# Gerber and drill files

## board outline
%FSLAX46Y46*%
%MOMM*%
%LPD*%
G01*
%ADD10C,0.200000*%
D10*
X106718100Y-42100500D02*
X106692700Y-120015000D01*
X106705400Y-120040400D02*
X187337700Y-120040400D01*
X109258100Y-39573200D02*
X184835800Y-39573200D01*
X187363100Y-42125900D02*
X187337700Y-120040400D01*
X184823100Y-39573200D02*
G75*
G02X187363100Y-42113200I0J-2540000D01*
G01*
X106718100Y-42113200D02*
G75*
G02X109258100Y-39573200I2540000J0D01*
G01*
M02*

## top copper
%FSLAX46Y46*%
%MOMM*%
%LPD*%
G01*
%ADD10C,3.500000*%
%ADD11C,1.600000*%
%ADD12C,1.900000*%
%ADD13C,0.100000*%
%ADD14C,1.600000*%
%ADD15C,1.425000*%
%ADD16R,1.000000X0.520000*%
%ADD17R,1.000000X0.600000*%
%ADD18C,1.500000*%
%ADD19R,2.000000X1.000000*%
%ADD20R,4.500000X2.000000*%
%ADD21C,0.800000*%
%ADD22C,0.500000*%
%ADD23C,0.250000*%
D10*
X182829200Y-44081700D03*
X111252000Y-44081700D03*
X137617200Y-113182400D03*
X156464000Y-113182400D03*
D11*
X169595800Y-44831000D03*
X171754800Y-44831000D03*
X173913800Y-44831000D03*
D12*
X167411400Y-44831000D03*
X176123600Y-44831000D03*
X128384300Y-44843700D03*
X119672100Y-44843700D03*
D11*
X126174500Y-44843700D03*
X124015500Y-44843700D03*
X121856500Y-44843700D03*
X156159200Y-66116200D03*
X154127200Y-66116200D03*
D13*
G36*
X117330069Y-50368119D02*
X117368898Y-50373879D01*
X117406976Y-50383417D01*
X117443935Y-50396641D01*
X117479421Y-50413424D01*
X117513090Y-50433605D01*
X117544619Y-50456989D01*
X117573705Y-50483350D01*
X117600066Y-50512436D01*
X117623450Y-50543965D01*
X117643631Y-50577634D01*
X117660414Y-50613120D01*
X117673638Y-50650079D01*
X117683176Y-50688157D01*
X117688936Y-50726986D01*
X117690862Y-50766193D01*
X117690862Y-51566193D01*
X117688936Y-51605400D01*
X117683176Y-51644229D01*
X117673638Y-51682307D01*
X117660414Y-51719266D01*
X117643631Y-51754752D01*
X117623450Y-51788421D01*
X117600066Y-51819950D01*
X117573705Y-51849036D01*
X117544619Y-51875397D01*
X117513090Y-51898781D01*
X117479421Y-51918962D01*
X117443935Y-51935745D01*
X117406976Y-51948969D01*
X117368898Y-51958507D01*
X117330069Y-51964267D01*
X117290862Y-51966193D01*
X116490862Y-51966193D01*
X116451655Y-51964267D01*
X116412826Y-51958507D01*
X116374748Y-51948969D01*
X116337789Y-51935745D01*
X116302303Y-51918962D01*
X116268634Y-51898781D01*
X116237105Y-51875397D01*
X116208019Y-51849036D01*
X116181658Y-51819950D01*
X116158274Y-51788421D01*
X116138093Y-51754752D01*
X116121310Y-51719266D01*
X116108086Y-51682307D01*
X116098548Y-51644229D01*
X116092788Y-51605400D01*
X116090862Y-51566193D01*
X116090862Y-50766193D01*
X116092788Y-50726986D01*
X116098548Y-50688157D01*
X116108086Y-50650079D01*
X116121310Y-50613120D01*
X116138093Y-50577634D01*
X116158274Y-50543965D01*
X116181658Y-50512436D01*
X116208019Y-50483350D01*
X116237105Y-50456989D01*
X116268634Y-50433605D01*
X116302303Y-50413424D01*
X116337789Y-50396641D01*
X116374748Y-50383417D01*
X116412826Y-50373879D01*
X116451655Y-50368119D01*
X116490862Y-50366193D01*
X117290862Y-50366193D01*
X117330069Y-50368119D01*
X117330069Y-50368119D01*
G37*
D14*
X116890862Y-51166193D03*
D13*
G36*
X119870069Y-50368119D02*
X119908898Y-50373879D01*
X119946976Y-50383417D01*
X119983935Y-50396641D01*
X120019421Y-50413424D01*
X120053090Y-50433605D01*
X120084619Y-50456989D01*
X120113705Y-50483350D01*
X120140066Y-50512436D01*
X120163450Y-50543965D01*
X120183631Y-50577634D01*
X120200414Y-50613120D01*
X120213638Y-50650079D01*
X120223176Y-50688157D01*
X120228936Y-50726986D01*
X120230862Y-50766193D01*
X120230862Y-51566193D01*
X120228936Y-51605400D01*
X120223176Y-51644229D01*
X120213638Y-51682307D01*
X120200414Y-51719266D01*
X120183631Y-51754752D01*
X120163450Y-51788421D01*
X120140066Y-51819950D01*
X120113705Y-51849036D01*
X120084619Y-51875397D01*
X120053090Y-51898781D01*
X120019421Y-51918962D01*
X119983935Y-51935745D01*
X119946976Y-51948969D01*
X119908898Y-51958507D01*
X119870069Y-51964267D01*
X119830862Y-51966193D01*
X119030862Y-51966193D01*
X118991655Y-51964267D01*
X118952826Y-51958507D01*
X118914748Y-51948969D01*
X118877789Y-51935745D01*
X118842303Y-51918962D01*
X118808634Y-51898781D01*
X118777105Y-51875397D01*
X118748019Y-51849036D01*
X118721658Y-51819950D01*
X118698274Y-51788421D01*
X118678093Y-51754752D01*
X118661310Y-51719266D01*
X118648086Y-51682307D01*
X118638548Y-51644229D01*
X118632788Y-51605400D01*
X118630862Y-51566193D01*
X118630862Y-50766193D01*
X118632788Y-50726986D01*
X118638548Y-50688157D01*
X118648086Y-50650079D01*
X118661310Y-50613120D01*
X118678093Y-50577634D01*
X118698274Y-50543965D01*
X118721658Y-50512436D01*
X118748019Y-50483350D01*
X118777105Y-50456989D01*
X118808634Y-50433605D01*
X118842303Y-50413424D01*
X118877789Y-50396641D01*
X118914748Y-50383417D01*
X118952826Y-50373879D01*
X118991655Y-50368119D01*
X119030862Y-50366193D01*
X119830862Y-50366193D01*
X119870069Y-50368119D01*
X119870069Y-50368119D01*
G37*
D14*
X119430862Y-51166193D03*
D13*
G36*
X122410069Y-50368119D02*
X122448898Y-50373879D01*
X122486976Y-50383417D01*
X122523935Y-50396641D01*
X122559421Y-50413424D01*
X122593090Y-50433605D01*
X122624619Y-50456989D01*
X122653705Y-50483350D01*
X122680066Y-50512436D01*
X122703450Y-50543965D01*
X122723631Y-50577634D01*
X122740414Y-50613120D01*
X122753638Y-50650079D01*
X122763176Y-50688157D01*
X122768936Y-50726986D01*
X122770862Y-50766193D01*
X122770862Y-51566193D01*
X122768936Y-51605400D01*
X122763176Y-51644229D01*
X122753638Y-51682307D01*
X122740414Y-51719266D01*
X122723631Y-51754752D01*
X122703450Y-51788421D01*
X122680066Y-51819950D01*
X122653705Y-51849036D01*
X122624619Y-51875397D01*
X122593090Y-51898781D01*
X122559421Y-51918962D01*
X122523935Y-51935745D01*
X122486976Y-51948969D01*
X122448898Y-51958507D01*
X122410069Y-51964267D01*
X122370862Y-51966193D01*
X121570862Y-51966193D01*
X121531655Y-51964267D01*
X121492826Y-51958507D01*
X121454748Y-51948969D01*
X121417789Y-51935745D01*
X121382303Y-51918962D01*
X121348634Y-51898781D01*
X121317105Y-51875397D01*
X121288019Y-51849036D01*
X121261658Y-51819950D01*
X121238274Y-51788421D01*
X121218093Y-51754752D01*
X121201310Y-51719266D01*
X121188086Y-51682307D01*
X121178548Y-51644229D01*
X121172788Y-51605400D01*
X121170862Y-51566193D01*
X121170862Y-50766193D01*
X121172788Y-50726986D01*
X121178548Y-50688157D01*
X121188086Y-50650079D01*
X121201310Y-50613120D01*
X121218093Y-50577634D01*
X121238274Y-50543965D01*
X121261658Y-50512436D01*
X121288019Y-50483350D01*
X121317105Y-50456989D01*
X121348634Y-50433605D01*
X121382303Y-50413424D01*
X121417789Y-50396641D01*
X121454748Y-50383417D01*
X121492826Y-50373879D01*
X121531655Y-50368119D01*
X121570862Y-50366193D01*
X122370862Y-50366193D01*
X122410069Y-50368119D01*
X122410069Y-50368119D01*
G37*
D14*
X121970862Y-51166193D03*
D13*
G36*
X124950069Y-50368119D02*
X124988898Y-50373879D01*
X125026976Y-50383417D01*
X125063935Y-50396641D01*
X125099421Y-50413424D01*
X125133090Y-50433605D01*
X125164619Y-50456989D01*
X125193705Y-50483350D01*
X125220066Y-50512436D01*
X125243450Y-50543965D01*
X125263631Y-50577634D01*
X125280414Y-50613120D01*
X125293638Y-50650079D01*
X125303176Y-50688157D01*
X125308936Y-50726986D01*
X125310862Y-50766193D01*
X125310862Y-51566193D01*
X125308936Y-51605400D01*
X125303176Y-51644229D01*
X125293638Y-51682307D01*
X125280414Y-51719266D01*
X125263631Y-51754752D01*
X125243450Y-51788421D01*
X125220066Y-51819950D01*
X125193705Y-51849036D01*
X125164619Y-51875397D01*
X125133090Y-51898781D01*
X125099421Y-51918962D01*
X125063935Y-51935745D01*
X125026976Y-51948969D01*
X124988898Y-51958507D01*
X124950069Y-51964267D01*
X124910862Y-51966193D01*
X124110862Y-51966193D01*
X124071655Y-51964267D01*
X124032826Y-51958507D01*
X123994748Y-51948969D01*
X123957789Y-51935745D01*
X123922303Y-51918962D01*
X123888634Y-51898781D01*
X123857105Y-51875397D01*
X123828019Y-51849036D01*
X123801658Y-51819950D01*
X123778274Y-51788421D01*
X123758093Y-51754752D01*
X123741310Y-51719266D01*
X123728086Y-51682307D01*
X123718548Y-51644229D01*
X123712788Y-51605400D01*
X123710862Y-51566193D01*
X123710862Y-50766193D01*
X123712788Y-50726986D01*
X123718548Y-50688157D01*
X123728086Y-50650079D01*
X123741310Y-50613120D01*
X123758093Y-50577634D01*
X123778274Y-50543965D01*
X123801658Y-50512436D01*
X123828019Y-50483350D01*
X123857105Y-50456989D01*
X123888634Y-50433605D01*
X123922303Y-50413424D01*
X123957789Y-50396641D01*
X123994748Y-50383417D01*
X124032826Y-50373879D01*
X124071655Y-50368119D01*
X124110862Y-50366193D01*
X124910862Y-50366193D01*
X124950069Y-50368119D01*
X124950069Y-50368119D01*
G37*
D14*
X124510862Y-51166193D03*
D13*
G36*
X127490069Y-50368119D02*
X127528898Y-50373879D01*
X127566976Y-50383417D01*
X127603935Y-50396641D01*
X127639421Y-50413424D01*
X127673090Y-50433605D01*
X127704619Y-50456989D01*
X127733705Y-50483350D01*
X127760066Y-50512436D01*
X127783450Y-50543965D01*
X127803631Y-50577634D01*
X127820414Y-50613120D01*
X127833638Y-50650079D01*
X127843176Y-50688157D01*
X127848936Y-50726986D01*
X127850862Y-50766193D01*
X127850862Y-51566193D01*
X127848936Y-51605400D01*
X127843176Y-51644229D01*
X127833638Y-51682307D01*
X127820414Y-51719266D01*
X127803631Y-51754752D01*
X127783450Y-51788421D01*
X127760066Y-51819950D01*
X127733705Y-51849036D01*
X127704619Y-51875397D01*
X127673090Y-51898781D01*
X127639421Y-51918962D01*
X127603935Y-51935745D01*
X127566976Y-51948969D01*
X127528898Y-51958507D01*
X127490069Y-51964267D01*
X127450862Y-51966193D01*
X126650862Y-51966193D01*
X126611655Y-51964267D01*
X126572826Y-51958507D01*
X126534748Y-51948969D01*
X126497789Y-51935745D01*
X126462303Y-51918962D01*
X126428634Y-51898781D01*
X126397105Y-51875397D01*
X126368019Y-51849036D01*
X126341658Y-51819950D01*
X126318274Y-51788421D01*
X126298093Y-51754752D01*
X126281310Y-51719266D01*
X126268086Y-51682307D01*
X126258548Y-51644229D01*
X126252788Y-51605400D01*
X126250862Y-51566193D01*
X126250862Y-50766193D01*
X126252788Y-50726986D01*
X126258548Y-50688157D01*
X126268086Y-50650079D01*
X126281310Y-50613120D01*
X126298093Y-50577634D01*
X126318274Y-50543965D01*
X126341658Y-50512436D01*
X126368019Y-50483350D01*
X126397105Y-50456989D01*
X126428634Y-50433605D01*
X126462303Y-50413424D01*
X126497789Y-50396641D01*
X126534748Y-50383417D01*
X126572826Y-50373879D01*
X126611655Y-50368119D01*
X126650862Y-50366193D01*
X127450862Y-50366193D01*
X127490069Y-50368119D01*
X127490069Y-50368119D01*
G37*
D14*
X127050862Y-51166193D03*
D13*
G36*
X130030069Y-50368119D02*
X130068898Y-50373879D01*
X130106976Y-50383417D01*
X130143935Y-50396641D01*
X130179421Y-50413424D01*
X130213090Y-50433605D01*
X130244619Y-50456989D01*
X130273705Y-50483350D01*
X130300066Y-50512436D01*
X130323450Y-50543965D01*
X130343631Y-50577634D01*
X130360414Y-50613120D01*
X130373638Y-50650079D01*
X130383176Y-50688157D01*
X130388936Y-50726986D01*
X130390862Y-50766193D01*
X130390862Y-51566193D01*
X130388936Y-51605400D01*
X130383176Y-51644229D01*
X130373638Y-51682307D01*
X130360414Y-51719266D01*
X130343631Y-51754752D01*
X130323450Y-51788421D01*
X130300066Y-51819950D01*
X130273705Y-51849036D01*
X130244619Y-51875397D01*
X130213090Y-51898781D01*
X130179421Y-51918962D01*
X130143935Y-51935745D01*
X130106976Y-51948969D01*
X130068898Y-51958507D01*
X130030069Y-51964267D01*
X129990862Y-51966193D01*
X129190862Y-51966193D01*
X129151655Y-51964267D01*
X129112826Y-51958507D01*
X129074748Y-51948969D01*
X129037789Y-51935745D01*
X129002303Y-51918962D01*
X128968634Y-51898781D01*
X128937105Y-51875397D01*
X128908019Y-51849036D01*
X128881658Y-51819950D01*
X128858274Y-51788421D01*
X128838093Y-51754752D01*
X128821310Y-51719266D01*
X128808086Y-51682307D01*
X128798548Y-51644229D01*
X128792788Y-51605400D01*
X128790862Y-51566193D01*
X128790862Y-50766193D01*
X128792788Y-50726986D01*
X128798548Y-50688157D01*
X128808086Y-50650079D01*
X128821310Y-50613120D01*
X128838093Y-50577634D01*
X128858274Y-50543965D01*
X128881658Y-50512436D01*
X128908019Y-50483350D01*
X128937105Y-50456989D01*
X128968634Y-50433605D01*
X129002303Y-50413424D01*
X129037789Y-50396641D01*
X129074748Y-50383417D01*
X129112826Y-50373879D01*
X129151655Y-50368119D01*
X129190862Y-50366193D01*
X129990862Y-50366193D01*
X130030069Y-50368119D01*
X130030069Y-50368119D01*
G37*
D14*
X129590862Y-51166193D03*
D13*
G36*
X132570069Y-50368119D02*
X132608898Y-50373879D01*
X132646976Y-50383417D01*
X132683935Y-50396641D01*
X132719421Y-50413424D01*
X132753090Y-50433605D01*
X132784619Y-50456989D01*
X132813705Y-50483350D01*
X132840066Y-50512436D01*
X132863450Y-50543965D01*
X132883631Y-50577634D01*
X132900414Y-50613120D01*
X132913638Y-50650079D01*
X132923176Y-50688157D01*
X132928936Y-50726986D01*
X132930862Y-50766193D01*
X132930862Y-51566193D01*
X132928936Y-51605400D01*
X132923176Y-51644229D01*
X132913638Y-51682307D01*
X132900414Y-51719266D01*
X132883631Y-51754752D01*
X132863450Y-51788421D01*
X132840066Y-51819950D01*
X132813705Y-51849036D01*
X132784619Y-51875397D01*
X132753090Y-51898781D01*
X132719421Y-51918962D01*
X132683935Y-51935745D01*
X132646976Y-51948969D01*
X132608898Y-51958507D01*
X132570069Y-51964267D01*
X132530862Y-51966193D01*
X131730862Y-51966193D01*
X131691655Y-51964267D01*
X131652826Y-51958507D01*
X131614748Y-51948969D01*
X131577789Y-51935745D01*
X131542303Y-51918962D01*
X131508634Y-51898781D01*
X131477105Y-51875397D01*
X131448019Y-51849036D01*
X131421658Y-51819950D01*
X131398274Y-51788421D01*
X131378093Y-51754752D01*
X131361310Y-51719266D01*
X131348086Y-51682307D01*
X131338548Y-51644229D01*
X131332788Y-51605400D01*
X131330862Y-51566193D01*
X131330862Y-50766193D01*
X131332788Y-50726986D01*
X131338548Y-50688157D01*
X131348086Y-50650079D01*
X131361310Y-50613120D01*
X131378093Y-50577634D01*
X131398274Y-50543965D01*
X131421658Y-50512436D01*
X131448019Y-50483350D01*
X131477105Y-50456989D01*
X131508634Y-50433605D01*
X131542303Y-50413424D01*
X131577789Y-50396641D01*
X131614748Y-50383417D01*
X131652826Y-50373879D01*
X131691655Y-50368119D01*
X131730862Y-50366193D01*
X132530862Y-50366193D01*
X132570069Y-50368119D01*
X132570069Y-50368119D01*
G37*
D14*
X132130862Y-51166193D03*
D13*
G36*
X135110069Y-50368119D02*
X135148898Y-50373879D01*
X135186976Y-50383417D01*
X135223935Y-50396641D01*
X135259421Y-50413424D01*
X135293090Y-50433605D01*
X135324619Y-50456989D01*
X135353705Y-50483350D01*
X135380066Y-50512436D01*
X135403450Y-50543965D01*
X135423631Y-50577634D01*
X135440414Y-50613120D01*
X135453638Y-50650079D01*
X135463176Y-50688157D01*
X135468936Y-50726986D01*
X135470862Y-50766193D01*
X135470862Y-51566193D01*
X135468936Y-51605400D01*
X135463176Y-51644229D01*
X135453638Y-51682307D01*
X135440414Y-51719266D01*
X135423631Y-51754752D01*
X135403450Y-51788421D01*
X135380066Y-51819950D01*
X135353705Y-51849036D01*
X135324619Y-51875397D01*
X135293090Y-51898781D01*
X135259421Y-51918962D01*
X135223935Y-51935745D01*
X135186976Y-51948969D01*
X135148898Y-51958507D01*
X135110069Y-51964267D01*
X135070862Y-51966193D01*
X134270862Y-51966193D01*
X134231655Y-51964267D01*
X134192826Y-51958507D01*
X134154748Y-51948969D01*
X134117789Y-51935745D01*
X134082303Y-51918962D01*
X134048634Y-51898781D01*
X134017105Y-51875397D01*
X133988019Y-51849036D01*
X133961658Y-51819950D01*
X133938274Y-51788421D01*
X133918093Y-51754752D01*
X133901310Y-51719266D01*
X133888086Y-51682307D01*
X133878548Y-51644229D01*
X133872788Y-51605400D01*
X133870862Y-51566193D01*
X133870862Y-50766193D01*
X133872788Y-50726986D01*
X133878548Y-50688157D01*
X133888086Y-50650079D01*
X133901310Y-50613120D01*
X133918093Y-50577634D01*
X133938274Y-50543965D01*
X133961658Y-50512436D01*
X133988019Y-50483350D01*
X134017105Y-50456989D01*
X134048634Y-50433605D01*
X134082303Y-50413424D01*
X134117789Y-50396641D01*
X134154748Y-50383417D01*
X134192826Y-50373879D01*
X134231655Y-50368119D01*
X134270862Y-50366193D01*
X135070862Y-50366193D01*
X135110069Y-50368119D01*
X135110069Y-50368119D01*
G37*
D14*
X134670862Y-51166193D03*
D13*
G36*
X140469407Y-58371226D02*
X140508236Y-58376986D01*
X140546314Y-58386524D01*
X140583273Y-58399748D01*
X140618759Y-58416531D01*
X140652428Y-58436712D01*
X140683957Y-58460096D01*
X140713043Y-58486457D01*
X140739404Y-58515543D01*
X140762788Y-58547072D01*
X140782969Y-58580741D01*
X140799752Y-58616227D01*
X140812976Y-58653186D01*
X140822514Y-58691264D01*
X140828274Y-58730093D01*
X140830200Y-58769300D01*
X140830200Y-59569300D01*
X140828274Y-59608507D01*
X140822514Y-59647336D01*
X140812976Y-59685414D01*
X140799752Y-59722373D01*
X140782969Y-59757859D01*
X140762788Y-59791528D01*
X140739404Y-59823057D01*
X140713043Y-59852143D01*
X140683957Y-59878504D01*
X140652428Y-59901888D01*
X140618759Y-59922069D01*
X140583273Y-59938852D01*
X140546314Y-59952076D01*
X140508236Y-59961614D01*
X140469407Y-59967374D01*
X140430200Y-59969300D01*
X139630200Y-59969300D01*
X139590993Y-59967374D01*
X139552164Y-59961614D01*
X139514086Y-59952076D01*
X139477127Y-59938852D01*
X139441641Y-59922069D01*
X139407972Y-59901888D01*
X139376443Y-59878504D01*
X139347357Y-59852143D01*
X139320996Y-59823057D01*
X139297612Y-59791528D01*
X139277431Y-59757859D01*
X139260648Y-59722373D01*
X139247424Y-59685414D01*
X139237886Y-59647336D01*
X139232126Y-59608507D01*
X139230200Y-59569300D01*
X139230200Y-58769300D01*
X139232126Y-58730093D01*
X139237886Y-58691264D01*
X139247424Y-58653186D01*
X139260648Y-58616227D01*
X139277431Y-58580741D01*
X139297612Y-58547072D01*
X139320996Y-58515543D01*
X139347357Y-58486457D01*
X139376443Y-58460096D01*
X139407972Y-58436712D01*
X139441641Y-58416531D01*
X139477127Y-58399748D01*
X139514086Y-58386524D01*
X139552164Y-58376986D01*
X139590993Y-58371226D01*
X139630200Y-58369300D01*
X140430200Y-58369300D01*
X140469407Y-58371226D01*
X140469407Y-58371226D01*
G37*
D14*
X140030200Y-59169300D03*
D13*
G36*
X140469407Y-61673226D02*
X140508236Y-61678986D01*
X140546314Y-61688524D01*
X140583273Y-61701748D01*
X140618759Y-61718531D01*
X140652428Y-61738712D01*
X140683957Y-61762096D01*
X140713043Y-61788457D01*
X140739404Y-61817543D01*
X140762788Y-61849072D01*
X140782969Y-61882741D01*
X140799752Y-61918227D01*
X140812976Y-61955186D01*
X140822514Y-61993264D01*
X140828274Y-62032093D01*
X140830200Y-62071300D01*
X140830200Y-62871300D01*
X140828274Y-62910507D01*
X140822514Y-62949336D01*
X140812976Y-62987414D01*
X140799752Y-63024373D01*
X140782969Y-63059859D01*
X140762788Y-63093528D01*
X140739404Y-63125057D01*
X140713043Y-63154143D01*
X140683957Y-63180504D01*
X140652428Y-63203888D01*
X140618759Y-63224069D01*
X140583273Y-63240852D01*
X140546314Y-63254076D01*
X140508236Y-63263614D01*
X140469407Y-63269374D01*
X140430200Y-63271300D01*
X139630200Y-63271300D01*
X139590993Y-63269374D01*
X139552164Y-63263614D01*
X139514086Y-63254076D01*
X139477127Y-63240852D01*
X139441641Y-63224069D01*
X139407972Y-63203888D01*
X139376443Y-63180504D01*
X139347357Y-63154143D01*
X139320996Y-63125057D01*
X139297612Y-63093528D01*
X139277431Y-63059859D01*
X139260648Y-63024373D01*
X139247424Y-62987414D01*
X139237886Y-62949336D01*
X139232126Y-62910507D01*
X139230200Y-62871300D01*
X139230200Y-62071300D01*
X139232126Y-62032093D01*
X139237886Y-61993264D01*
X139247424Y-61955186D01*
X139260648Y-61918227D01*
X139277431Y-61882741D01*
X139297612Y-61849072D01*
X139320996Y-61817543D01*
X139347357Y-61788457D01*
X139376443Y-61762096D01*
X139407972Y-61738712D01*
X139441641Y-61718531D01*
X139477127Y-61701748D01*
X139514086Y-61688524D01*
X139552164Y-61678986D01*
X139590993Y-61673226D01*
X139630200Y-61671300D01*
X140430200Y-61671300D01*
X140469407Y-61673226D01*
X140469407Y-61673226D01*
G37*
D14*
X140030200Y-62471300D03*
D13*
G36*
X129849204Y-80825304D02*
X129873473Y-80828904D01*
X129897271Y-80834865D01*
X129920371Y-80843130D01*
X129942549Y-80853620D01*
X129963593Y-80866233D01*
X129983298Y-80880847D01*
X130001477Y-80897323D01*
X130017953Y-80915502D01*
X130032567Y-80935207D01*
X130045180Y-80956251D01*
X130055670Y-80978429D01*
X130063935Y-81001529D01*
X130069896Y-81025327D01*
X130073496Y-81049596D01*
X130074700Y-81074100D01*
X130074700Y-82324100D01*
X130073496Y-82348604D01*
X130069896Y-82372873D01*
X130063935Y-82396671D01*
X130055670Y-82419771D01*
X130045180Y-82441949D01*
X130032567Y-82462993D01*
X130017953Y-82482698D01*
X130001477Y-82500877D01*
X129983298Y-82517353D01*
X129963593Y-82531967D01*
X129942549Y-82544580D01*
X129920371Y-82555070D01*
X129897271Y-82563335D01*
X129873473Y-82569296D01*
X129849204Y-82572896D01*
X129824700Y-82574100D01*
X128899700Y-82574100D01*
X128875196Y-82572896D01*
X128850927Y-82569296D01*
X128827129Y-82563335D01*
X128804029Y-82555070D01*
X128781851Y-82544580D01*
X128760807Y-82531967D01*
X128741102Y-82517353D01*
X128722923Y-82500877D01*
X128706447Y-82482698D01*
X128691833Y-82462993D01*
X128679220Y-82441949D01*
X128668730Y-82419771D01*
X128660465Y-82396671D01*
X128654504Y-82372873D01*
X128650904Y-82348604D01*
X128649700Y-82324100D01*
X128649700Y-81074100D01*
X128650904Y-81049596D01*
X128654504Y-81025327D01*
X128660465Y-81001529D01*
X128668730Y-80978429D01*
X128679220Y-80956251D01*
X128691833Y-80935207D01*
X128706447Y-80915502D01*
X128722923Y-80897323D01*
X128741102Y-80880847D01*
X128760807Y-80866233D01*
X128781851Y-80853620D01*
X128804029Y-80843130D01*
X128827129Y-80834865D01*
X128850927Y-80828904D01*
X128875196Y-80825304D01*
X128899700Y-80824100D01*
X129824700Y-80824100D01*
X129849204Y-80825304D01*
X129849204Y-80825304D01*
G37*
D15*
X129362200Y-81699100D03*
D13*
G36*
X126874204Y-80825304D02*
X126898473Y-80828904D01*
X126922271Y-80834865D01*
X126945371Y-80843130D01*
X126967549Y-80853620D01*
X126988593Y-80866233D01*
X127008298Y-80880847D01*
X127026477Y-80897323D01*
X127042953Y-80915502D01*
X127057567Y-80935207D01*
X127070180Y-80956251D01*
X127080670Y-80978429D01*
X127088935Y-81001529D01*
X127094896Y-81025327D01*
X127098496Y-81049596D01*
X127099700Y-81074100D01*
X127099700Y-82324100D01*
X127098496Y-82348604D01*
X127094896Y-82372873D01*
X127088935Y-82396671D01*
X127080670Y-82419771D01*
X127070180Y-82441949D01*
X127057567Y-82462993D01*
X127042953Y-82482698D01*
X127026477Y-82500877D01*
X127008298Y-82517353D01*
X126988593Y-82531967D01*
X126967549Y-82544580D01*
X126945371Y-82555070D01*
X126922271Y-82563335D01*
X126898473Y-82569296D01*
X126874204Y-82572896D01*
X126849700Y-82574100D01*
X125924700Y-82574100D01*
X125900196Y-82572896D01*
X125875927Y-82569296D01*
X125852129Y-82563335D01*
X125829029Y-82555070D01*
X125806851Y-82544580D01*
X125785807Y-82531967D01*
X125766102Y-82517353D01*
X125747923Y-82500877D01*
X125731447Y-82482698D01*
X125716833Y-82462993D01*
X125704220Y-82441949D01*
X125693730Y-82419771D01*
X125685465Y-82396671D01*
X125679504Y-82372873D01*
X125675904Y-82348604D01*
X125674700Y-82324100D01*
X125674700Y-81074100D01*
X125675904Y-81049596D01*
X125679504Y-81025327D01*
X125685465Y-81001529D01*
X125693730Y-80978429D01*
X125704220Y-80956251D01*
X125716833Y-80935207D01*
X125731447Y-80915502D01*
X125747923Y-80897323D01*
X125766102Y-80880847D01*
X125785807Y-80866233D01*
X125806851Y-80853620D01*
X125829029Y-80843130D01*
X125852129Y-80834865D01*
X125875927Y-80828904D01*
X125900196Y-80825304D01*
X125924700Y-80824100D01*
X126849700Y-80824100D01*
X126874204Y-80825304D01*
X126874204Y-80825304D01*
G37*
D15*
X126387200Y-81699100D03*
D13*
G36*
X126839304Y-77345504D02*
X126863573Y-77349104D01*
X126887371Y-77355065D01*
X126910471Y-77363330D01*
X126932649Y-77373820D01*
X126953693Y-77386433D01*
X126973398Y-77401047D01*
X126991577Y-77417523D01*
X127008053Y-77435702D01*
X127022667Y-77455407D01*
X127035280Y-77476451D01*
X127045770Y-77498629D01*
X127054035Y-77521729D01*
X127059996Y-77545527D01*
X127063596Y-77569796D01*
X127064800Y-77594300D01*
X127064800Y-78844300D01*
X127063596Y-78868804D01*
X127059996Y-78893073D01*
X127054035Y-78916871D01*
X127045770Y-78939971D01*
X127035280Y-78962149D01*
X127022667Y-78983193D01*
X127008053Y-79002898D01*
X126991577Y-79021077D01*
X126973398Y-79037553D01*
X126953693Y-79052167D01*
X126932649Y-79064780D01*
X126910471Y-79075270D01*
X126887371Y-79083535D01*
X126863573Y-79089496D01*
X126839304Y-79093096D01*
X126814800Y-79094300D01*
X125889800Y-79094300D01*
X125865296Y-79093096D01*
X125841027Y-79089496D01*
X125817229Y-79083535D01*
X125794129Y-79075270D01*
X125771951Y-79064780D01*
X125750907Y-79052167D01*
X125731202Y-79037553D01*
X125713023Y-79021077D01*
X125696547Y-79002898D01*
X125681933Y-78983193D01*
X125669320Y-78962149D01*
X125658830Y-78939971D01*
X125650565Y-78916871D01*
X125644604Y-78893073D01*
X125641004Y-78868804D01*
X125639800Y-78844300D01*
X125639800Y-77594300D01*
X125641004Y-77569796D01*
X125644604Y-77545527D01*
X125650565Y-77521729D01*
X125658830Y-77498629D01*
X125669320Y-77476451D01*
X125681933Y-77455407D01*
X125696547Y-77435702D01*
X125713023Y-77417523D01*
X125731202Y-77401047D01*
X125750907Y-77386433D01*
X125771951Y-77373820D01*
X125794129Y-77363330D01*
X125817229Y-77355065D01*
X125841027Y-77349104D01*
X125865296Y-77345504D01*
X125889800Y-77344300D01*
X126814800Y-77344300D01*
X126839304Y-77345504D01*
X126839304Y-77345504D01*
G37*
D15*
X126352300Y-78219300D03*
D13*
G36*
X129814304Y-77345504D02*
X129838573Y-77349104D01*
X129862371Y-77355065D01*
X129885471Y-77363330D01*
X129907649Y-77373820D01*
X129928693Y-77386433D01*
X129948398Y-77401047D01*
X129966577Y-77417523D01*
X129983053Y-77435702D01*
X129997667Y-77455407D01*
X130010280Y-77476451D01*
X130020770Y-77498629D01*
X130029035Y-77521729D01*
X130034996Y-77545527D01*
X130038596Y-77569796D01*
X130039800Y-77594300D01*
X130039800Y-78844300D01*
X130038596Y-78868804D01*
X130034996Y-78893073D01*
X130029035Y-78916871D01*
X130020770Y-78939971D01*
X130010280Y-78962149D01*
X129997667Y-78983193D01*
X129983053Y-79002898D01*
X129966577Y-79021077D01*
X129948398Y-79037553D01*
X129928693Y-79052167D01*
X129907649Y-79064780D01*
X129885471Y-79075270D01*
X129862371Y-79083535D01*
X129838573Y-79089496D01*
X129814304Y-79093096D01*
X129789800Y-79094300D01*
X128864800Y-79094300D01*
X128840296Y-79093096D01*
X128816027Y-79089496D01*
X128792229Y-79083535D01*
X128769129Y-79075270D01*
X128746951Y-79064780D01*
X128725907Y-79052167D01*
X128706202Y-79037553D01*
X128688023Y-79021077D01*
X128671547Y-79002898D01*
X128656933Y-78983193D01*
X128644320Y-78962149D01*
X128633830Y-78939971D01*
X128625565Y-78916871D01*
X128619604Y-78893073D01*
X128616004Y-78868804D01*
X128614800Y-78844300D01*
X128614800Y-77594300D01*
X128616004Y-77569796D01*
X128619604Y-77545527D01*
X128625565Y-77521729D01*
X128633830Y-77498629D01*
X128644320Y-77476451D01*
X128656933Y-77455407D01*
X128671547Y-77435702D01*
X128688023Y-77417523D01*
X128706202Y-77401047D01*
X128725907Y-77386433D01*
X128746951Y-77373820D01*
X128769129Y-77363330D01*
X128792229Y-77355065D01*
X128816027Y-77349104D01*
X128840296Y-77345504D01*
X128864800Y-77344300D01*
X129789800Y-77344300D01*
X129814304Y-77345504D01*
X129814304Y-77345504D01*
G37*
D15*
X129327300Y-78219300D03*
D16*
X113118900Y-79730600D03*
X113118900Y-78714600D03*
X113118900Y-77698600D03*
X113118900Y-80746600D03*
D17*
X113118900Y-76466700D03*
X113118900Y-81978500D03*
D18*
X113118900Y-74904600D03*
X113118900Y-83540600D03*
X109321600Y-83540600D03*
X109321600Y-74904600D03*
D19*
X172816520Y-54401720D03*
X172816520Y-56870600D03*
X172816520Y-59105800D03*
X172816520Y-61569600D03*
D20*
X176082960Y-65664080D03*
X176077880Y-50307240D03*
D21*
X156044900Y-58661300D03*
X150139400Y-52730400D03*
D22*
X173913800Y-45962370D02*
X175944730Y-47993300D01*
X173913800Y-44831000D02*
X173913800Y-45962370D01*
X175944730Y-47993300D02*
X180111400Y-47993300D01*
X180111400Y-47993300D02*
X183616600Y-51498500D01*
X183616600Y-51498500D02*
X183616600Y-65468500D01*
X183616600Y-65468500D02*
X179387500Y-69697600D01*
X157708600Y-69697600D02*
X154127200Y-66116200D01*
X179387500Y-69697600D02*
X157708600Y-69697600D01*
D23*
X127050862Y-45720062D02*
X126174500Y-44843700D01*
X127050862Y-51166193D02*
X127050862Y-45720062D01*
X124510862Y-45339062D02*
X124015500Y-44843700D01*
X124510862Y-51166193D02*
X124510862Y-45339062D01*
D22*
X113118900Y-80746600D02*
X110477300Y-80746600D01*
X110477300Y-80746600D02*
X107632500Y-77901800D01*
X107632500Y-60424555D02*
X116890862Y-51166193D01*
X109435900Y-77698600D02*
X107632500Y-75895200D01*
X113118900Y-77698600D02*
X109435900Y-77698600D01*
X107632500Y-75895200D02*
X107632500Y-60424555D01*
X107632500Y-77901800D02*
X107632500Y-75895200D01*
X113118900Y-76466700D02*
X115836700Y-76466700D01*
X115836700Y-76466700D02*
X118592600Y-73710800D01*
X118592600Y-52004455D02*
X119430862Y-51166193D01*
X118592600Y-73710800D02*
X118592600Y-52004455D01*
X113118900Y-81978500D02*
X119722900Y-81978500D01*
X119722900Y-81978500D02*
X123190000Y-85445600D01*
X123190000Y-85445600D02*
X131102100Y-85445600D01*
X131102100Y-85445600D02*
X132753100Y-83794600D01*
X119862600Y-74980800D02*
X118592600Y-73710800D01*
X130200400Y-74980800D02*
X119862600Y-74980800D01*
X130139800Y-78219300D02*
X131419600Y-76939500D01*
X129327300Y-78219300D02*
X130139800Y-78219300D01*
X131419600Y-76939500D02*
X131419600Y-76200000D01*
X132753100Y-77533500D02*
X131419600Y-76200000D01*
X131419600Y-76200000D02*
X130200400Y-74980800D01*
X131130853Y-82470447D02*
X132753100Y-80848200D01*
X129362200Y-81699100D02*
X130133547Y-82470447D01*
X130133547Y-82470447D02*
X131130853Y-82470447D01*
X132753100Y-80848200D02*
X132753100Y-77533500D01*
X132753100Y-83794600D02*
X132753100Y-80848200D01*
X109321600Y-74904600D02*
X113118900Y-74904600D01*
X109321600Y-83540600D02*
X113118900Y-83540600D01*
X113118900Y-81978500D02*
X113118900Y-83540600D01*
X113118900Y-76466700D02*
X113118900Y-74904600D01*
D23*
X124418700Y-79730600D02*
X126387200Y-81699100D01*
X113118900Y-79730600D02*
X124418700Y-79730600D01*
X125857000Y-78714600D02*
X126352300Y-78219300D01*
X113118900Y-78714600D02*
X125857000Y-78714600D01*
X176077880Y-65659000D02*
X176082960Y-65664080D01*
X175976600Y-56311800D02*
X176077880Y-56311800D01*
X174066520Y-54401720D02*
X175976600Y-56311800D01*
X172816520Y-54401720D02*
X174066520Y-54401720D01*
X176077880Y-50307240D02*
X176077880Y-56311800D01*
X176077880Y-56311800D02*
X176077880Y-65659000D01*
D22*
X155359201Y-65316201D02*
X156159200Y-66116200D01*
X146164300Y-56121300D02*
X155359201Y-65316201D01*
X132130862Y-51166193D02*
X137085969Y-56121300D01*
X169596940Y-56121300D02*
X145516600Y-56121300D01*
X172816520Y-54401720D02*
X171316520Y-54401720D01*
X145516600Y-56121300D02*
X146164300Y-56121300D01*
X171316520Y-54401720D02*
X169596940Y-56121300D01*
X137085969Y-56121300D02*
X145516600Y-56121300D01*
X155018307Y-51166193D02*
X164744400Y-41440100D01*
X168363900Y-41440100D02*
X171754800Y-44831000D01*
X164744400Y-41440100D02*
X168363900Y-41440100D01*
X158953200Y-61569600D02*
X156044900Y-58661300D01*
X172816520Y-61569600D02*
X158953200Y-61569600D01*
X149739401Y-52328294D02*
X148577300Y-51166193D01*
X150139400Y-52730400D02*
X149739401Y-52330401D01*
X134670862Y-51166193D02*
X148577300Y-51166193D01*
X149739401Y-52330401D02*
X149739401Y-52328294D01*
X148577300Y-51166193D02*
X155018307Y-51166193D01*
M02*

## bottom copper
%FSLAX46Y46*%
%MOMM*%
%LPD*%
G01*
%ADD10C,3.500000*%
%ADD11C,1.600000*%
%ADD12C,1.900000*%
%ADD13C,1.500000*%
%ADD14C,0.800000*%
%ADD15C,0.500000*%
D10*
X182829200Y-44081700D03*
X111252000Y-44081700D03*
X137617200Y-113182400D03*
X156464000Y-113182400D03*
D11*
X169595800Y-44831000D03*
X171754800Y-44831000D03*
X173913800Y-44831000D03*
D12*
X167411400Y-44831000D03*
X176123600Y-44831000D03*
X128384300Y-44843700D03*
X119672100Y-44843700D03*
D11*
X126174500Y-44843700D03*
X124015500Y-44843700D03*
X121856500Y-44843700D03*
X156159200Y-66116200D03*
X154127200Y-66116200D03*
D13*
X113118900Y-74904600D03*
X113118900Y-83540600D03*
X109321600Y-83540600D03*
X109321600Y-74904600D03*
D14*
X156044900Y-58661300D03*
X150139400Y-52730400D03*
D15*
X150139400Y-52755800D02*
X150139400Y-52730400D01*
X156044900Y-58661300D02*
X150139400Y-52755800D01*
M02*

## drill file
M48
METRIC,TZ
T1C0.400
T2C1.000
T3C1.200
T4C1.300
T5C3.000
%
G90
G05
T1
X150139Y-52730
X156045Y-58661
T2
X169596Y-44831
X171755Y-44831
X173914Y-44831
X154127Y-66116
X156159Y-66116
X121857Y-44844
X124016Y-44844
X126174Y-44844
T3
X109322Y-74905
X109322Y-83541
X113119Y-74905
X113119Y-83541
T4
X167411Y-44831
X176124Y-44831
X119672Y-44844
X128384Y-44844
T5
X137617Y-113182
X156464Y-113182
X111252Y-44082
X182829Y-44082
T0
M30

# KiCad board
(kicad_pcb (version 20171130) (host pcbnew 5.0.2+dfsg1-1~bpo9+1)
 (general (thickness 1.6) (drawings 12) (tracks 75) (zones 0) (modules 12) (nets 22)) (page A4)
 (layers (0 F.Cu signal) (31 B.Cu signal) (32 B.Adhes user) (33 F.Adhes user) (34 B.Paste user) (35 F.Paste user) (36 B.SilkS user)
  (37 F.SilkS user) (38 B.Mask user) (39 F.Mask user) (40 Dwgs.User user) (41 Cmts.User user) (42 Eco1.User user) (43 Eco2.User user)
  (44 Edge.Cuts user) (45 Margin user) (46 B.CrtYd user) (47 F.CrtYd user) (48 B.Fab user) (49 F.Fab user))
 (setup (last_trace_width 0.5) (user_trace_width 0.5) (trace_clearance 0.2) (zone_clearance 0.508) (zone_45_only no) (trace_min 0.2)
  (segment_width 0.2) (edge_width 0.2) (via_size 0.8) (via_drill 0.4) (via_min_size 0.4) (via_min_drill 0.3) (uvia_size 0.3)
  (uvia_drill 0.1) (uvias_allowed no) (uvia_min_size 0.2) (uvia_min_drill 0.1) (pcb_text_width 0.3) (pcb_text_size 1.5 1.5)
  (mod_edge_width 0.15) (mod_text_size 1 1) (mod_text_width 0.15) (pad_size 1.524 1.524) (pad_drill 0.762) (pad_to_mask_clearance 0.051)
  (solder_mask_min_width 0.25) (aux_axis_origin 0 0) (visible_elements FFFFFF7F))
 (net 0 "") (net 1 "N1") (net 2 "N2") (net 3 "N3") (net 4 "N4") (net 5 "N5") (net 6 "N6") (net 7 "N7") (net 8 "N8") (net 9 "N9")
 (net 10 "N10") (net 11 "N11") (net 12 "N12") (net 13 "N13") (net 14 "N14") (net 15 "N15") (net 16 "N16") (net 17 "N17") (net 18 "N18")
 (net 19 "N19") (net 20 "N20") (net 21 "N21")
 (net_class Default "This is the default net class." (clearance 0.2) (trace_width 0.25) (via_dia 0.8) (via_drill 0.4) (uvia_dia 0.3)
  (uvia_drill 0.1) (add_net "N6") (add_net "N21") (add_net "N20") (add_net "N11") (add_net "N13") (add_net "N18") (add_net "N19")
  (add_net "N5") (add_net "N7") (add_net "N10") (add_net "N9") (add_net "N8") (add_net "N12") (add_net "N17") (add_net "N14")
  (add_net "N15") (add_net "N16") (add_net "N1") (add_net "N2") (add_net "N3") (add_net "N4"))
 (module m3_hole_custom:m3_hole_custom (layer F.Cu) (at 182.8292 44.0817)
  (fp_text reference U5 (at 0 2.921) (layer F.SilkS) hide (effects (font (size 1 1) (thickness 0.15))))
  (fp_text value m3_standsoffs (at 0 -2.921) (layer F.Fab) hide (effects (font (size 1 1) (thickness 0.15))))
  (pad 1 thru_hole circle (at 0 0) (size 3.5 3.5) (drill 3) (layers *.Cu *.Mask) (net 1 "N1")))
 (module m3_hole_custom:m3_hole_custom (layer F.Cu) (at 111.252 44.0817)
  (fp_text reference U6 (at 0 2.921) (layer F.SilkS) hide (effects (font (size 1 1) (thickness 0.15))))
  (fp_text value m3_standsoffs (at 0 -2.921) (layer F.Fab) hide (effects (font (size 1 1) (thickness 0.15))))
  (pad 1 thru_hole circle (at 0 0) (size 3.5 3.5) (drill 3) (layers *.Cu *.Mask) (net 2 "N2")))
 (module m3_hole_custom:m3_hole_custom (layer F.Cu) (at 137.6172 113.1824)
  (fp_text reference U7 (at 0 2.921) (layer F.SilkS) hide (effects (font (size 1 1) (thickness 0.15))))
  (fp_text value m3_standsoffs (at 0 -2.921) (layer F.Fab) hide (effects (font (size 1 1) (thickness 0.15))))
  (pad 1 thru_hole circle (at 0 0) (size 3.5 3.5) (drill 3) (layers *.Cu *.Mask) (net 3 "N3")))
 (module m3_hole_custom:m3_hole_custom (layer F.Cu) (at 156.464 113.1824)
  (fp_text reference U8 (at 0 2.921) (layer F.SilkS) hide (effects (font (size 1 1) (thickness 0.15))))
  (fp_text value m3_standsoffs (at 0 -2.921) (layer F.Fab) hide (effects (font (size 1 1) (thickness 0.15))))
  (pad 1 thru_hole circle (at 0 0) (size 3.5 3.5) (drill 3) (layers *.Cu *.Mask) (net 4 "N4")))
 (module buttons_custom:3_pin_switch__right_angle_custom (layer F.Cu) (at 171.7548 44.831)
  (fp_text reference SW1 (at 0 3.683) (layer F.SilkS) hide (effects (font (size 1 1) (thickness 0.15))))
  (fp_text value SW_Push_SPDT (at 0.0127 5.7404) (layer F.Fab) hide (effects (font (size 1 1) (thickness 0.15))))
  (pad 1 thru_hole circle (at -2.159 0) (size 1.6 1.6) (drill 1) (layers *.Cu *.Mask) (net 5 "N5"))
  (pad 2 thru_hole circle (at 0 0) (size 1.6 1.6) (drill 1) (layers *.Cu *.Mask) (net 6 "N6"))
  (pad 3 thru_hole circle (at 2.159 0) (size 1.6 1.6) (drill 1) (layers *.Cu *.Mask) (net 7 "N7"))
  (pad 4 thru_hole circle (at -4.3434 0) (size 1.9 1.9) (drill 1.3) (layers *.Cu *.Mask))
  (pad 4 thru_hole circle (at 4.3688 0) (size 1.9 1.9) (drill 1.3) (layers *.Cu *.Mask)))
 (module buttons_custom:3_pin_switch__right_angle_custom (layer F.Cu) (at 124.0155 44.8437)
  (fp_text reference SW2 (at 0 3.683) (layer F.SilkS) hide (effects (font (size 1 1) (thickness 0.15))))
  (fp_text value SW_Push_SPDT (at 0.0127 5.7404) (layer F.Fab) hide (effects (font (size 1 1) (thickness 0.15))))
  (pad 4 thru_hole circle (at 4.3688 0) (size 1.9 1.9) (drill 1.3) (layers *.Cu *.Mask))
  (pad 4 thru_hole circle (at -4.3434 0) (size 1.9 1.9) (drill 1.3) (layers *.Cu *.Mask))
  (pad 3 thru_hole circle (at 2.159 0) (size 1.6 1.6) (drill 1) (layers *.Cu *.Mask) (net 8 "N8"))
  (pad 2 thru_hole circle (at 0 0) (size 1.6 1.6) (drill 1) (layers *.Cu *.Mask) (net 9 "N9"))
  (pad 1 thru_hole circle (at -2.159 0) (size 1.6 1.6) (drill 1) (layers *.Cu *.Mask) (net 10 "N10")))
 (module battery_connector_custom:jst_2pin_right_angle (layer F.Cu) (at 155.1432 66.1162 180)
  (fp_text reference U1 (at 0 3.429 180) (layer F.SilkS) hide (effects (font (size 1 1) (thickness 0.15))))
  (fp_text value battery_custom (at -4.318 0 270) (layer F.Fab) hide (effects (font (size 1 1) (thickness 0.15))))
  (pad 1 thru_hole circle (at -1.016 0 180) (size 1.6 1.6) (drill 1) (layers *.Cu *.Mask) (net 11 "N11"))
  (pad 2 thru_hole circle (at 1.016 0 180) (size 1.6 1.6) (drill 1) (layers *.Cu *.Mask) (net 7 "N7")))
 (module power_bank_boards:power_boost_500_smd (layer F.Cu) (at 142.3162 60.6933 90)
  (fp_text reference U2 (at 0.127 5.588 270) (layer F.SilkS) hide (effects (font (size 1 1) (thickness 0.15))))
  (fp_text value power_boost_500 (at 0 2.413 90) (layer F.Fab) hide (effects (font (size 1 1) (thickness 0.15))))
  (pad 1 smd roundrect (at 9.527107 -25.425338 270) (size 1.6 1.6) (layers F.Cu F.Paste F.Mask) (roundrect_rratio 0.25) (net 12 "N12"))
  (pad 2 smd roundrect (at 9.527107 -22.885338 270) (size 1.6 1.6) (layers F.Cu F.Paste F.Mask) (roundrect_rratio 0.25) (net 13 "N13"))
  (pad 3 smd roundrect (at 9.527107 -20.345338 270) (size 1.6 1.6) (layers F.Cu F.Paste F.Mask) (roundrect_rratio 0.25) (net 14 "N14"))
  (pad 4 smd roundrect (at 9.527107 -17.805338 270) (size 1.6 1.6) (layers F.Cu F.Paste F.Mask) (roundrect_rratio 0.25) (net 9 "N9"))
  (pad 5 smd roundrect (at 9.527107 -15.265338 270) (size 1.6 1.6) (layers F.Cu F.Paste F.Mask) (roundrect_rratio 0.25) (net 8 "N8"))
  (pad 6 smd roundrect (at 9.527107 -12.725338 270) (size 1.6 1.6) (layers F.Cu F.Paste F.Mask) (roundrect_rratio 0.25) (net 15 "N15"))
  (pad 7 smd roundrect (at 9.527107 -10.185338 270) (size 1.6 1.6) (layers F.Cu F.Paste F.Mask) (roundrect_rratio 0.25) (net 11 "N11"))
  (pad 8 smd roundrect (at 9.527107 -7.645338 270) (size 1.6 1.6) (layers F.Cu F.Paste F.Mask) (roundrect_rratio 0.25) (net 6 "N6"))
  (pad 9 smd roundrect (at 1.524 -2.286 270) (size 1.6 1.6) (layers F.Cu F.Paste F.Mask) (roundrect_rratio 0.25) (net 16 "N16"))
  (pad 10 smd roundrect (at -1.778 -2.286 270) (size 1.6 1.6) (layers F.Cu F.Paste F.Mask) (roundrect_rratio 0.25) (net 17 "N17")))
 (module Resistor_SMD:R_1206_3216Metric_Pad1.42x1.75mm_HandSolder (layer F.Cu) (at 127.8747 81.6991 180)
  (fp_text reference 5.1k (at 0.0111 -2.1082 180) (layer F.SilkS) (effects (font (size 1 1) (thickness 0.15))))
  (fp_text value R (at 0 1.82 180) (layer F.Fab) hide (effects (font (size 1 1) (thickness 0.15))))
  (pad 1 smd roundrect (at -1.4875 0 180) (size 1.425 1.75) (layers F.Cu F.Paste F.Mask) (roundrect_rratio 0.175439) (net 13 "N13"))
  (pad 2 smd roundrect (at 1.4875 0 180) (size 1.425 1.75) (layers F.Cu F.Paste F.Mask) (roundrect_rratio 0.175439) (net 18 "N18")))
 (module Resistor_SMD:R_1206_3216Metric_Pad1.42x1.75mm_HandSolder (layer F.Cu) (at 127.8398 78.2193 180)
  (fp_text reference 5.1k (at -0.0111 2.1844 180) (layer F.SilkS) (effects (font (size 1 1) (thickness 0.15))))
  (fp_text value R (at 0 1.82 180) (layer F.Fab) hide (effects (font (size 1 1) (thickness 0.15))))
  (pad 2 smd roundrect (at 1.4875 0 180) (size 1.425 1.75) (layers F.Cu F.Paste F.Mask) (roundrect_rratio 0.175439) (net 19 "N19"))
  (pad 1 smd roundrect (at -1.4875 0 180) (size 1.425 1.75) (layers F.Cu F.Paste F.Mask) (roundrect_rratio 0.175439) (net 13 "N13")))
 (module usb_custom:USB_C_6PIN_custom (layer F.Cu) (at 113.1189 79.2226 90)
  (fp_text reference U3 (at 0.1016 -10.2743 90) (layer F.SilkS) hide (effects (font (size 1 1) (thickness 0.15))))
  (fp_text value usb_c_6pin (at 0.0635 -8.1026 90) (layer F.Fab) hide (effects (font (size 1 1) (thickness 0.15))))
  (pad 3 smd rect (at -0.508 0 90) (size 0.52 1) (layers F.Cu F.Paste F.Mask) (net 18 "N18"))
  (pad 4 smd rect (at 0.508 0 90) (size 0.52 1) (layers F.Cu F.Paste F.Mask) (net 19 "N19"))
  (pad 2 smd rect (at 1.524 0 90) (size 0.52 1) (layers F.Cu F.Paste F.Mask) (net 12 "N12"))
  (pad 2 smd rect (at -1.524 0 90) (size 0.52 1) (layers F.Cu F.Paste F.Mask) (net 12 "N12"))
  (pad 1 smd rect (at 2.7559 0 90) (size 0.6 1) (layers F.Cu F.Paste F.Mask) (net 13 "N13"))
  (pad 1 smd rect (at -2.7559 0 90) (size 0.6 1) (layers F.Cu F.Paste F.Mask) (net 13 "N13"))
  (pad 1 thru_hole circle (at 4.318 0 90) (size 1.5 1.5) (drill 1.2) (layers *.Cu *.Mask) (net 13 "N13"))
  (pad 1 thru_hole circle (at -4.318 0 90) (size 1.5 1.5) (drill 1.2) (layers *.Cu *.Mask) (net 13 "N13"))
  (pad 1 thru_hole circle (at -4.318 -3.7973 90) (size 1.5 1.5) (drill 1.2) (layers *.Cu *.Mask) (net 13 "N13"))
  (pad 1 thru_hole circle (at 4.318 -3.7973 90) (size 1.5 1.5) (drill 1.2) (layers *.Cu *.Mask) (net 13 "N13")))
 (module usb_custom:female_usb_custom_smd (layer F.Cu) (at 174.7774 57.9882 270)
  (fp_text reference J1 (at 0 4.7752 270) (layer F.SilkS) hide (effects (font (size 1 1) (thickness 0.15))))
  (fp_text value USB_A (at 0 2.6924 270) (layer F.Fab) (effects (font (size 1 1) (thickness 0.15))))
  (pad 4 smd rect (at -3.58648 1.96088 270) (size 1 2) (layers F.Cu F.Paste F.Mask) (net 11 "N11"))
  (pad 3 smd rect (at -1.1176 1.96088 270) (size 1 2) (layers F.Cu F.Paste F.Mask) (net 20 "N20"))
  (pad 2 smd rect (at 1.1176 1.96088 270) (size 1 2) (layers F.Cu F.Paste F.Mask) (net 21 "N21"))
  (pad 1 smd rect (at 3.5814 1.96088 270) (size 1 2) (layers F.Cu F.Paste F.Mask) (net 6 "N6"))
  (pad 5 smd rect (at 7.67588 -1.30556 270) (size 2 4.5) (layers F.Cu F.Paste F.Mask) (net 11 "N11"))
  (pad 5 smd rect (at -7.68096 -1.30048 270) (size 2 4.5) (layers F.Cu F.Paste F.Mask) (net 11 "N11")))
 (gr_line (start 106.7181 42.1005) (end 106.6927 120.015) (layer Edge.Cuts) (width 0.2))
 (gr_line (start 106.7054 120.0404) (end 187.3377 120.0404) (layer Edge.Cuts) (width 0.2))
 (gr_line (start 109.2581 39.5732) (end 184.8358 39.5732) (layer Edge.Cuts) (width 0.2))
 (gr_line (start 187.3631 42.1259) (end 187.3377 120.0404) (layer Edge.Cuts) (width 0.2))
 (gr_arc (start 184.8231 42.1132) (end 187.3631 42.1132) (angle -90) (layer Edge.Cuts) (width 0.2))
 (gr_arc (start 109.2581 42.1132) (end 109.2581 39.5732) (angle -90) (layer Edge.Cuts) (width 0.2))
 (segment (start 173.9138 45.96237) (end 175.94473 47.9933) (width 0.5) (layer F.Cu) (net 7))
 (segment (start 173.9138 44.831) (end 173.9138 45.96237) (width 0.5) (layer F.Cu) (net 7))
 (segment (start 175.94473 47.9933) (end 180.1114 47.9933) (width 0.5) (layer F.Cu) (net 7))
 (segment (start 180.1114 47.9933) (end 183.6166 51.4985) (width 0.5) (layer F.Cu) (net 7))
 (segment (start 183.6166 51.4985) (end 183.6166 65.4685) (width 0.5) (layer F.Cu) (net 7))
 (segment (start 183.6166 65.4685) (end 179.3875 69.6976) (width 0.5) (layer F.Cu) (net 7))
 (segment (start 157.7086 69.6976) (end 154.1272 66.1162) (width 0.5) (layer F.Cu) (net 7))
 (segment (start 179.3875 69.6976) (end 157.7086 69.6976) (width 0.5) (layer F.Cu) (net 7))
 (segment (start 127.050862 45.720062) (end 126.1745 44.8437) (width 0.25) (layer F.Cu) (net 8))
 (segment (start 127.050862 51.166193) (end 127.050862 45.720062) (width 0.25) (layer F.Cu) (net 8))
 (segment (start 124.510862 45.339062) (end 124.0155 44.8437) (width 0.25) (layer F.Cu) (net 9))
 (segment (start 124.510862 51.166193) (end 124.510862 45.339062) (width 0.25) (layer F.Cu) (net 9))
 (segment (start 113.1189 80.7466) (end 110.4773 80.7466) (width 0.5) (layer F.Cu) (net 12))
 (segment (start 110.4773 80.7466) (end 107.6325 77.9018) (width 0.5) (layer F.Cu) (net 12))
 (segment (start 107.6325 60.424555) (end 116.890862 51.166193) (width 0.5) (layer F.Cu) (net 12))
 (segment (start 109.4359 77.6986) (end 107.6325 75.8952) (width 0.5) (layer F.Cu) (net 12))
 (segment (start 113.1189 77.6986) (end 109.4359 77.6986) (width 0.5) (layer F.Cu) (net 12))
 (segment (start 107.6325 75.8952) (end 107.6325 60.424555) (width 0.5) (layer F.Cu) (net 12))
 (segment (start 107.6325 77.9018) (end 107.6325 75.8952) (width 0.5) (layer F.Cu) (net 12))
 (segment (start 113.1189 76.4667) (end 115.8367 76.4667) (width 0.5) (layer F.Cu) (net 13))
 (segment (start 115.8367 76.4667) (end 118.5926 73.7108) (width 0.5) (layer F.Cu) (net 13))
 (segment (start 118.5926 52.004455) (end 119.430862 51.166193) (width 0.5) (layer F.Cu) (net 13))
 (segment (start 118.5926 73.7108) (end 118.5926 52.004455) (width 0.5) (layer F.Cu) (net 13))
 (segment (start 113.1189 81.9785) (end 119.7229 81.9785) (width 0.5) (layer F.Cu) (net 13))
 (segment (start 119.7229 81.9785) (end 123.19 85.4456) (width 0.5) (layer F.Cu) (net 13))
 (segment (start 123.19 85.4456) (end 131.1021 85.4456) (width 0.5) (layer F.Cu) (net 13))
 (segment (start 131.1021 85.4456) (end 132.7531 83.7946) (width 0.5) (layer F.Cu) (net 13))
 (segment (start 119.8626 74.9808) (end 118.5926 73.7108) (width 0.5) (layer F.Cu) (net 13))
 (segment (start 130.2004 74.9808) (end 119.8626 74.9808) (width 0.5) (layer F.Cu) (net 13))
 (segment (start 130.1398 78.2193) (end 131.4196 76.9395) (width 0.5) (layer F.Cu) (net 13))
 (segment (start 129.3273 78.2193) (end 130.1398 78.2193) (width 0.5) (layer F.Cu) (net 13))
 (segment (start 131.4196 76.9395) (end 131.4196 76.2) (width 0.5) (layer F.Cu) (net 13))
 (segment (start 132.7531 77.5335) (end 131.4196 76.2) (width 0.5) (layer F.Cu) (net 13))
 (segment (start 131.4196 76.2) (end 130.2004 74.9808) (width 0.5) (layer F.Cu) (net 13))
 (segment (start 131.130853 82.470447) (end 132.7531 80.8482) (width 0.5) (layer F.Cu) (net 13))
 (segment (start 129.3622 81.6991) (end 130.133547 82.470447) (width 0.5) (layer F.Cu) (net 13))
 (segment (start 130.133547 82.470447) (end 131.130853 82.470447) (width 0.5) (layer F.Cu) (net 13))
 (segment (start 132.7531 80.8482) (end 132.7531 77.5335) (width 0.5) (layer F.Cu) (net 13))
 (segment (start 132.7531 83.7946) (end 132.7531 80.8482) (width 0.5) (layer F.Cu) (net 13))
 (segment (start 109.3216 74.9046) (end 113.1189 74.9046) (width 0.5) (layer F.Cu) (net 13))
 (segment (start 109.3216 83.5406) (end 113.1189 83.5406) (width 0.5) (layer F.Cu) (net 13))
 (segment (start 113.1189 81.9785) (end 113.1189 83.5406) (width 0.5) (layer F.Cu) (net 13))
 (segment (start 113.1189 76.4667) (end 113.1189 74.9046) (width 0.5) (layer F.Cu) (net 13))
 (segment (start 124.4187 79.7306) (end 126.3872 81.6991) (width 0.25) (layer F.Cu) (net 18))
 (segment (start 113.1189 79.7306) (end 124.4187 79.7306) (width 0.25) (layer F.Cu) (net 18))
 (segment (start 125.857 78.7146) (end 126.3523 78.2193) (width 0.25) (layer F.Cu) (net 19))
 (segment (start 113.1189 78.7146) (end 125.857 78.7146) (width 0.25) (layer F.Cu) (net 19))
 (segment (start 176.07788 65.659) (end 176.08296 65.66408) (width 0.25) (layer F.Cu) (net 11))
 (segment (start 175.9766 56.3118) (end 176.07788 56.3118) (width 0.25) (layer F.Cu) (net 11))
 (segment (start 174.06652 54.40172) (end 175.9766 56.3118) (width 0.25) (layer F.Cu) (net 11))
 (segment (start 172.81652 54.40172) (end 174.06652 54.40172) (width 0.25) (layer F.Cu) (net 11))
 (segment (start 176.07788 50.30724) (end 176.07788 56.3118) (width 0.25) (layer F.Cu) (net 11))
 (segment (start 176.07788 56.3118) (end 176.07788 65.659) (width 0.25) (layer F.Cu) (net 11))
 (segment (start 155.359201 65.316201) (end 156.1592 66.1162) (width 0.5) (layer F.Cu) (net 11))
 (segment (start 146.1643 56.1213) (end 155.359201 65.316201) (width 0.5) (layer F.Cu) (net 11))
 (segment (start 132.130862 51.166193) (end 137.085969 56.1213) (width 0.5) (layer F.Cu) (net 11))
 (segment (start 169.59694 56.1213) (end 145.5166 56.1213) (width 0.5) (layer F.Cu) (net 11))
 (segment (start 172.81652 54.40172) (end 171.31652 54.40172) (width 0.5) (layer F.Cu) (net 11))
 (segment (start 145.5166 56.1213) (end 146.1643 56.1213) (width 0.5) (layer F.Cu) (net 11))
 (segment (start 171.31652 54.40172) (end 169.59694 56.1213) (width 0.5) (layer F.Cu) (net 11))
 (segment (start 137.085969 56.1213) (end 145.5166 56.1213) (width 0.5) (layer F.Cu) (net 11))
 (segment (start 155.018307 51.166193) (end 164.7444 41.4401) (width 0.5) (layer F.Cu) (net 6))
 (segment (start 168.3639 41.4401) (end 171.7548 44.831) (width 0.5) (layer F.Cu) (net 6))
 (segment (start 164.7444 41.4401) (end 168.3639 41.4401) (width 0.5) (layer F.Cu) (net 6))
 (via (at 156.0449 58.6613) (size 0.8) (drill 0.4) (layers F.Cu B.Cu) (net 6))
 (segment (start 158.9532 61.5696) (end 156.0449 58.6613) (width 0.5) (layer F.Cu) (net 6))
 (segment (start 172.81652 61.5696) (end 158.9532 61.5696) (width 0.5) (layer F.Cu) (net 6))
 (via (at 150.1394 52.7304) (size 0.8) (drill 0.4) (layers F.Cu B.Cu) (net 6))
 (segment (start 150.1394 52.7558) (end 150.1394 52.7304) (width 0.5) (layer B.Cu) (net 6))
 (segment (start 156.0449 58.6613) (end 150.1394 52.7558) (width 0.5) (layer B.Cu) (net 6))
 (segment (start 149.739401 52.328294) (end 148.5773 51.166193) (width 0.5) (layer F.Cu) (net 6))
 (segment (start 150.1394 52.7304) (end 149.739401 52.330401) (width 0.5) (layer F.Cu) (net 6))
 (segment (start 134.670862 51.166193) (end 148.5773 51.166193) (width 0.5) (layer F.Cu) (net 6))
 (segment (start 149.739401 52.330401) (end 149.739401 52.328294) (width 0.5) (layer F.Cu) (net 6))
 (segment (start 148.5773 51.166193) (end 155.018307 51.166193) (width 0.5) (layer F.Cu) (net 6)))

